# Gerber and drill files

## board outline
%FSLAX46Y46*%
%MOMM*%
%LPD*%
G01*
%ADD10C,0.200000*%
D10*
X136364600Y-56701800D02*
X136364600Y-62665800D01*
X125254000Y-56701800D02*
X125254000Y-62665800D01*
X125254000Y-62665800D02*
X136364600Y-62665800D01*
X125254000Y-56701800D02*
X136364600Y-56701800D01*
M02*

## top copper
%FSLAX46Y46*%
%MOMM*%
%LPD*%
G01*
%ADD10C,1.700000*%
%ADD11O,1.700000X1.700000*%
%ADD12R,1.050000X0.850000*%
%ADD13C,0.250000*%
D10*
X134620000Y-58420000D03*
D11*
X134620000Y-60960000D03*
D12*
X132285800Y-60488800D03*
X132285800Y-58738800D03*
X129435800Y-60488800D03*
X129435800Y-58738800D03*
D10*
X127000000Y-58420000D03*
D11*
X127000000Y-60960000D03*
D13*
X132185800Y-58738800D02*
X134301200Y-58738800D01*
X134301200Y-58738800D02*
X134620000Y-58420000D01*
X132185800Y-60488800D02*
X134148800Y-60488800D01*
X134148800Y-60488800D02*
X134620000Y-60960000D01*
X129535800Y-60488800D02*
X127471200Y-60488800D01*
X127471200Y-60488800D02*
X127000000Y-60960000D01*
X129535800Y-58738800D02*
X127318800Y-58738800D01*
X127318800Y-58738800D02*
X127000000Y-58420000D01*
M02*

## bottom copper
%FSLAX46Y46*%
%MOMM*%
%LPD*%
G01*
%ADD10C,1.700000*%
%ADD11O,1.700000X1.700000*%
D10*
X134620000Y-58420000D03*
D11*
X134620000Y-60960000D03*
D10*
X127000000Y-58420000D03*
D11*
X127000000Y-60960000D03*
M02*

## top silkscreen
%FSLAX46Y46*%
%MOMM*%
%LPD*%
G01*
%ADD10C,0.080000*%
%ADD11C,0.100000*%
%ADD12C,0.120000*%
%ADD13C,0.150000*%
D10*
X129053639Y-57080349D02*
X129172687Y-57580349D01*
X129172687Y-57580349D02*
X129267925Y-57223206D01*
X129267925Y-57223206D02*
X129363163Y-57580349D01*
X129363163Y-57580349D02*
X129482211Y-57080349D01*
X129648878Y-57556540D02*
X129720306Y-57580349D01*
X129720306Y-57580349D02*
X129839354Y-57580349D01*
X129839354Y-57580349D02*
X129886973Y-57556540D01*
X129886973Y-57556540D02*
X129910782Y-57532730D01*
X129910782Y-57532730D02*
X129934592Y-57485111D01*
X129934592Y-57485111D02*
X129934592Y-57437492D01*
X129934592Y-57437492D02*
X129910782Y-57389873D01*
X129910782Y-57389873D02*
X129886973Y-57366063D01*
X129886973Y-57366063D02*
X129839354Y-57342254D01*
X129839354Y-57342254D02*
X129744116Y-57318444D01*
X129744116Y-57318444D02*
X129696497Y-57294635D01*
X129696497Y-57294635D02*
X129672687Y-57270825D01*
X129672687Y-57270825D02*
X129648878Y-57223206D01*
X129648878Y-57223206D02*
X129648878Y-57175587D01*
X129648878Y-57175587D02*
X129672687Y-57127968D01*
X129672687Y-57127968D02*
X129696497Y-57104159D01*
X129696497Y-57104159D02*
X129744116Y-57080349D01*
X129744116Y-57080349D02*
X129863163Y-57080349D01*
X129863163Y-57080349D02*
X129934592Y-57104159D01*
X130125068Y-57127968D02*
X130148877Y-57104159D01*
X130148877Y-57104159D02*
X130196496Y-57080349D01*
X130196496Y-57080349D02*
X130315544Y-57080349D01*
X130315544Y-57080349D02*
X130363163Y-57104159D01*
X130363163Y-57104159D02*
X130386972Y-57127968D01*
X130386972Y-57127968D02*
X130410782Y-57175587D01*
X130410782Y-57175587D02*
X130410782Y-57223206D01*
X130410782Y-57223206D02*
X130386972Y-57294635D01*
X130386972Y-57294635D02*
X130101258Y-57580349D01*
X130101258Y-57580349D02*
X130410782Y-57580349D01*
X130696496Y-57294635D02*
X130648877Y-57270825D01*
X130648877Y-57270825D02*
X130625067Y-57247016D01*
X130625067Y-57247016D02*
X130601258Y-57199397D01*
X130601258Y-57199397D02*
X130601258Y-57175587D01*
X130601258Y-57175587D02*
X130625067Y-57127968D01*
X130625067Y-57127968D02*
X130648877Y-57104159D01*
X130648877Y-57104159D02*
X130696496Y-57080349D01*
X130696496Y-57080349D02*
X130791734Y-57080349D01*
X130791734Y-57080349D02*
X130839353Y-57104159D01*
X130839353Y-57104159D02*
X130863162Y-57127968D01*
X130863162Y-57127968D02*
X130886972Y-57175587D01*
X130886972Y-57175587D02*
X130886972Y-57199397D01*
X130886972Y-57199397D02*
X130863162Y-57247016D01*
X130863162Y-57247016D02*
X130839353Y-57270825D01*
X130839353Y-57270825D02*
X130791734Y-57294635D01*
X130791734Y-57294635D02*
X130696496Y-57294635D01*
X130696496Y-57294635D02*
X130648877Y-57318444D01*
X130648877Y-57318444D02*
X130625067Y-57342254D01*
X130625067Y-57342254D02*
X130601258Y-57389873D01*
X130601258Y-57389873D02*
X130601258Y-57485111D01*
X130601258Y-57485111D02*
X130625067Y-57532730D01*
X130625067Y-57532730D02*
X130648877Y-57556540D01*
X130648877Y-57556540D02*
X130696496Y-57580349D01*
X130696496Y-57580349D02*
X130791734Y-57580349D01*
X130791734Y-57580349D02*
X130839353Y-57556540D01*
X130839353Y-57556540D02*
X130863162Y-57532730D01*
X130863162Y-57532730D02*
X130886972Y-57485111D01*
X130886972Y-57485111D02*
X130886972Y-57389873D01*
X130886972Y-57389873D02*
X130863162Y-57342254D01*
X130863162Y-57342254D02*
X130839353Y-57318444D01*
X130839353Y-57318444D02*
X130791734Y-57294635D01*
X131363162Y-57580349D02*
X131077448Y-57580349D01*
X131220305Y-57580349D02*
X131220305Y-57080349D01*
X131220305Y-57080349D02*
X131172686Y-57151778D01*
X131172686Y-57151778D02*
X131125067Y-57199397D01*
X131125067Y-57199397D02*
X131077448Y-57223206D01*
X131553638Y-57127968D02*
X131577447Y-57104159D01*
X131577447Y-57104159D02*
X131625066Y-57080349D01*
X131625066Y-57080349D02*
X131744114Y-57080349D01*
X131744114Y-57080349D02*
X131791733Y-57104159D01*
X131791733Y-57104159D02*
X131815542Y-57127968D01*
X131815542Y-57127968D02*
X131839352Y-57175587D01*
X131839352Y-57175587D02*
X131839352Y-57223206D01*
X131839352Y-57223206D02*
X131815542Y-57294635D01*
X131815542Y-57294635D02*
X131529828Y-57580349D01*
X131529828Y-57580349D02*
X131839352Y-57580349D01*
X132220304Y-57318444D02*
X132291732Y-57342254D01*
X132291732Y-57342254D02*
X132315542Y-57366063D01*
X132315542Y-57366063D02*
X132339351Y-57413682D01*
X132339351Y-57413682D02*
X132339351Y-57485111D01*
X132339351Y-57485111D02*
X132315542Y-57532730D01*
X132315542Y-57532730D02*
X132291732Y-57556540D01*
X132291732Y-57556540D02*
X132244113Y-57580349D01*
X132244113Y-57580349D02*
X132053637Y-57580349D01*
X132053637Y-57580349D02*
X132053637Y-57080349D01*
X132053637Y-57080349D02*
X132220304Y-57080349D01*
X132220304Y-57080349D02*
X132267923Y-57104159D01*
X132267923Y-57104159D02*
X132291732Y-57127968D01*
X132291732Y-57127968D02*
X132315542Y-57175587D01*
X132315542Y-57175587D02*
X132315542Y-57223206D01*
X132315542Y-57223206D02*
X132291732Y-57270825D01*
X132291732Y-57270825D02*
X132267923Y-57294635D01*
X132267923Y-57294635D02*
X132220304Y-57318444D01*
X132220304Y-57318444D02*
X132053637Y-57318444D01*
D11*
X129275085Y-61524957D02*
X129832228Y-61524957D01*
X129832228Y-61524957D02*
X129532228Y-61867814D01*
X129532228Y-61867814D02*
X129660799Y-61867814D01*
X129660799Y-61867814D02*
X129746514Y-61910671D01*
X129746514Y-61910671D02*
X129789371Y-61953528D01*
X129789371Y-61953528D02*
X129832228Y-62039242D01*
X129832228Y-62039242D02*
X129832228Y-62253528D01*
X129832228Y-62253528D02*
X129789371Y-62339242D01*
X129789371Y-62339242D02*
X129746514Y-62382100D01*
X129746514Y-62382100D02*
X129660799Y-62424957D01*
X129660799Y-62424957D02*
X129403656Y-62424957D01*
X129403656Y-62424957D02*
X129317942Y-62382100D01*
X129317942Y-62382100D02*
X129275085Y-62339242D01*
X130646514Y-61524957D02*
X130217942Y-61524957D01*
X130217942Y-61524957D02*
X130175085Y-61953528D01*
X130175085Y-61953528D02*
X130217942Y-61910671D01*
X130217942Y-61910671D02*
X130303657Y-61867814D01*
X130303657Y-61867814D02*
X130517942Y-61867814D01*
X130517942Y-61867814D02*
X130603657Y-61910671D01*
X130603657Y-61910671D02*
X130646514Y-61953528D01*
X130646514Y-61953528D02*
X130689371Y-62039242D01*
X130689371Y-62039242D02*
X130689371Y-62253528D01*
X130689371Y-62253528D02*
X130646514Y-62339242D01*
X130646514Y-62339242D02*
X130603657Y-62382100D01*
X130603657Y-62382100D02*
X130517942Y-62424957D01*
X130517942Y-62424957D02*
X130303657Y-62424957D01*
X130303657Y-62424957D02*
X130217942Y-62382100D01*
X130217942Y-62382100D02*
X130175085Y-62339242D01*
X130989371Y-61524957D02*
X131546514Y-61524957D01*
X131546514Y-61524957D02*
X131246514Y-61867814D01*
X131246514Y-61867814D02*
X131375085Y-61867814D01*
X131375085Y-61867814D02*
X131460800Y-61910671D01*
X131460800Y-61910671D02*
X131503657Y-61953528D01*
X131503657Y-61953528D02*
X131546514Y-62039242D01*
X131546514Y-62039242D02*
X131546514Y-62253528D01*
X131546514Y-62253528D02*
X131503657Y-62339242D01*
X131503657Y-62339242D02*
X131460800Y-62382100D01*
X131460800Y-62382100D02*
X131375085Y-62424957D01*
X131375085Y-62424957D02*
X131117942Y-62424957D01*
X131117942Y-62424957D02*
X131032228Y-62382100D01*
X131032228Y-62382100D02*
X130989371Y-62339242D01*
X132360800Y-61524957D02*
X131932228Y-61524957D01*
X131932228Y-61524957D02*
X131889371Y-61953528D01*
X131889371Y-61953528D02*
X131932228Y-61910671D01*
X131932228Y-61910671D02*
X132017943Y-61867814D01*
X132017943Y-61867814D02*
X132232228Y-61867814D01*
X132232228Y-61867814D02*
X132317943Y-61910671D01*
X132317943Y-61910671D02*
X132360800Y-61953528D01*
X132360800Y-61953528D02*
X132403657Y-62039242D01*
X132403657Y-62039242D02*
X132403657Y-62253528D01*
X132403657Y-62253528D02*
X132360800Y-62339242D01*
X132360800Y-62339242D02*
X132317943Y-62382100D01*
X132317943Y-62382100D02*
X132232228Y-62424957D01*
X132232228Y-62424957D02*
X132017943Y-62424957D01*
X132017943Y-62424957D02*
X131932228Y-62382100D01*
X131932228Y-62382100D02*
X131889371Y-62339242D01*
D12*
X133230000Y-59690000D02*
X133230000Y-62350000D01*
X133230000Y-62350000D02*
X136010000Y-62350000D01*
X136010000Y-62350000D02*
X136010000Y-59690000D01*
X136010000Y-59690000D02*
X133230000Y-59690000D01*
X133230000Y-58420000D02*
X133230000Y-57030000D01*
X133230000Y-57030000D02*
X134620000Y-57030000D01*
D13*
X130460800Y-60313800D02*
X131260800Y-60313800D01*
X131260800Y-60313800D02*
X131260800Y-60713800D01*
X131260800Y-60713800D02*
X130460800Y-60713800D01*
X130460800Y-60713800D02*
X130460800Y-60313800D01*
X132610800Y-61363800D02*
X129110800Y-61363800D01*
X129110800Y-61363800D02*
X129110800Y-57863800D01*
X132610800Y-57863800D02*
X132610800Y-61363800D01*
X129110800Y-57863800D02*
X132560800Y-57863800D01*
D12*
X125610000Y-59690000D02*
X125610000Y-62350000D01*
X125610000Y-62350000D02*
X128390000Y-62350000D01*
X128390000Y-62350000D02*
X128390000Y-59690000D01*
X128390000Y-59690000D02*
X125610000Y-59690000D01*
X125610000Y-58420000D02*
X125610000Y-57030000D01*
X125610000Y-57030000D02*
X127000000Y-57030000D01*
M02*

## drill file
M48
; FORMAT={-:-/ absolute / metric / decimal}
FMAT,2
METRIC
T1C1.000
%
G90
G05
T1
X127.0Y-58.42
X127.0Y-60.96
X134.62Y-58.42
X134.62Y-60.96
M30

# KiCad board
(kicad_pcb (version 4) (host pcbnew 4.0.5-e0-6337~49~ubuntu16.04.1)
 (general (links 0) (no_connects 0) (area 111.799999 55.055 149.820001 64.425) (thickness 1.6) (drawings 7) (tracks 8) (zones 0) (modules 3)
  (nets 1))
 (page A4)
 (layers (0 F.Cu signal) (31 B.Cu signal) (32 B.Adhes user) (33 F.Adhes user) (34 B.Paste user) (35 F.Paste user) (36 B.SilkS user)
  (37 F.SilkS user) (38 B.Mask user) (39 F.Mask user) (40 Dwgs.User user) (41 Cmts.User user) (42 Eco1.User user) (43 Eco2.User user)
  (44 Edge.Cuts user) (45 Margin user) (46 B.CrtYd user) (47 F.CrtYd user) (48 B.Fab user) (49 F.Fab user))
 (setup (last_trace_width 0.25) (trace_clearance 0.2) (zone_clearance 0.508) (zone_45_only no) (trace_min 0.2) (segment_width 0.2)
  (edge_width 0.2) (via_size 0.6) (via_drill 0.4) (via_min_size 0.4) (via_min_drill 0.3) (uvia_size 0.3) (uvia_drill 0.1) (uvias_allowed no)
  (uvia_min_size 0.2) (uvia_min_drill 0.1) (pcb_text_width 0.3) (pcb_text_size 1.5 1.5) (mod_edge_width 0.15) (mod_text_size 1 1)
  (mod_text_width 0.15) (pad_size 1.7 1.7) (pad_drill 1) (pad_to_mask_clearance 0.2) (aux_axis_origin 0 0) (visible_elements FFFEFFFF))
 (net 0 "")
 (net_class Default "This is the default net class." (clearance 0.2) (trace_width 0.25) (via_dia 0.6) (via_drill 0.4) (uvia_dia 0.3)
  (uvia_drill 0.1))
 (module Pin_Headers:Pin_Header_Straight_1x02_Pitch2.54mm (layer F.Cu) (at 134.62 58.42)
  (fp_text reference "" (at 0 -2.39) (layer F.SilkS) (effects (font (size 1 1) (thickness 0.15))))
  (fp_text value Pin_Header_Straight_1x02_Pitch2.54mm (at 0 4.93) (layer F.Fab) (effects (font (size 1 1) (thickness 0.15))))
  (fp_line (start -1.39 1.27) (end -1.39 3.93) (layer F.SilkS) (width 0.12))
  (fp_line (start -1.39 3.93) (end 1.39 3.93) (layer F.SilkS) (width 0.12))
  (fp_line (start 1.39 3.93) (end 1.39 1.27) (layer F.SilkS) (width 0.12))
  (fp_line (start 1.39 1.27) (end -1.39 1.27) (layer F.SilkS) (width 0.12))
  (fp_line (start -1.39 0) (end -1.39 -1.39) (layer F.SilkS) (width 0.12))
  (fp_line (start -1.39 -1.39) (end 0 -1.39) (layer F.SilkS) (width 0.12))
  (pad 1 thru_hole circle (at 0 0) (size 1.7 1.7) (drill 1) (layers *.Cu *.Mask))
  (pad 2 thru_hole oval (at 0 2.54) (size 1.7 1.7) (drill 1) (layers *.Cu *.Mask)))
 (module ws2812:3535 (layer F.Cu) (at 130.8608 59.6138)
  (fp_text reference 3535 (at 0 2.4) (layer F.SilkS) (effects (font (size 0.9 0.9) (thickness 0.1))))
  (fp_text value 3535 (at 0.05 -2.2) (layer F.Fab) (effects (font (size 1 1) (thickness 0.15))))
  (fp_line (start -0.4 0.7) (end 0.4 0.7) (layer F.SilkS) (width 0.15))
  (fp_line (start 0.4 0.7) (end 0.4 1.1) (layer F.SilkS) (width 0.15))
  (fp_line (start 0.4 1.1) (end -0.4 1.1) (layer F.SilkS) (width 0.15))
  (fp_line (start -0.4 1.1) (end -0.4 0.7) (layer F.SilkS) (width 0.15))
  (fp_line (start 1.75 1.75) (end -1.75 1.75) (layer F.SilkS) (width 0.15))
  (fp_line (start -1.75 1.75) (end -1.75 -1.75) (layer F.SilkS) (width 0.15))
  (fp_line (start 1.75 -1.75) (end 1.75 1.75) (layer F.SilkS) (width 0.15))
  (fp_line (start -1.75 -1.75) (end 1.7 -1.75) (layer F.SilkS) (width 0.15))
  (pad IN smd rect (at 1.325 0.875) (size 1.05 0.85) (drill (offset 0.1 0)) (layers F.Cu F.Paste F.Mask))
  (pad VDD smd rect (at 1.325 -0.875) (size 1.05 0.85) (drill (offset 0.1 0)) (layers F.Cu F.Paste F.Mask))
  (pad GND smd rect (at -1.325 0.875) (size 1.05 0.85) (drill (offset -0.1 0)) (layers F.Cu F.Paste F.Mask))
  (pad OUT smd rect (at -1.325 -0.875) (size 1.05 0.85) (drill (offset -0.1 0)) (layers F.Cu F.Paste F.Mask)))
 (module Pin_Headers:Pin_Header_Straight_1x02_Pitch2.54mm (layer F.Cu) (at 127 58.42)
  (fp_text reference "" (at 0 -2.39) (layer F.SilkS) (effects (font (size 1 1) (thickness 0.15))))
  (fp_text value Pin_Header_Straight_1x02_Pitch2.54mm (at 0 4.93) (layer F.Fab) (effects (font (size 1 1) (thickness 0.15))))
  (fp_line (start -1.39 1.27) (end -1.39 3.93) (layer F.SilkS) (width 0.12))
  (fp_line (start -1.39 3.93) (end 1.39 3.93) (layer F.SilkS) (width 0.12))
  (fp_line (start 1.39 3.93) (end 1.39 1.27) (layer F.SilkS) (width 0.12))
  (fp_line (start 1.39 1.27) (end -1.39 1.27) (layer F.SilkS) (width 0.12))
  (fp_line (start -1.39 0) (end -1.39 -1.39) (layer F.SilkS) (width 0.12))
  (fp_line (start -1.39 -1.39) (end 0 -1.39) (layer F.SilkS) (width 0.12))
  (pad 1 thru_hole circle (at 0 0) (size 1.7 1.7) (drill 1) (layers *.Cu *.Mask))
  (pad 2 thru_hole oval (at 0 2.54) (size 1.7 1.7) (drill 1) (layers *.Cu *.Mask)))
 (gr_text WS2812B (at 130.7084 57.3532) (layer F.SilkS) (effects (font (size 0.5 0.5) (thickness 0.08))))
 (gr_line (start 136.3646 56.7018) (end 136.3646 62.6658) (angle 90) (layer Edge.Cuts) (width 0.2))
 (gr_line (start 125.254 56.7018) (end 125.254 62.6658) (angle 90) (layer Edge.Cuts) (width 0.2))
 (gr_line (start 125.254 62.6658) (end 136.3646 62.6658) (angle 90) (layer Edge.Cuts) (width 0.2))
 (gr_line (start 125.254 56.7018) (end 136.3646 56.7018) (angle 90) (layer Edge.Cuts) (width 0.2))
 (segment (start 132.1858 58.7388) (end 134.3012 58.7388) (width 0.25) (layer F.Cu) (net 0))
 (segment (start 134.3012 58.7388) (end 134.62 58.42) (width 0.25) (layer F.Cu) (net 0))
 (segment (start 132.1858 60.4888) (end 134.1488 60.4888) (width 0.25) (layer F.Cu) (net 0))
 (segment (start 134.1488 60.4888) (end 134.62 60.96) (width 0.25) (layer F.Cu) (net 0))
 (segment (start 129.5358 60.4888) (end 127.4712 60.4888) (width 0.25) (layer F.Cu) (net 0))
 (segment (start 127.4712 60.4888) (end 127 60.96) (width 0.25) (layer F.Cu) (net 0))
 (segment (start 129.5358 58.7388) (end 127.3188 58.7388) (width 0.25) (layer F.Cu) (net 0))
 (segment (start 127.3188 58.7388) (end 127 58.42) (width 0.25) (layer F.Cu) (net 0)))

